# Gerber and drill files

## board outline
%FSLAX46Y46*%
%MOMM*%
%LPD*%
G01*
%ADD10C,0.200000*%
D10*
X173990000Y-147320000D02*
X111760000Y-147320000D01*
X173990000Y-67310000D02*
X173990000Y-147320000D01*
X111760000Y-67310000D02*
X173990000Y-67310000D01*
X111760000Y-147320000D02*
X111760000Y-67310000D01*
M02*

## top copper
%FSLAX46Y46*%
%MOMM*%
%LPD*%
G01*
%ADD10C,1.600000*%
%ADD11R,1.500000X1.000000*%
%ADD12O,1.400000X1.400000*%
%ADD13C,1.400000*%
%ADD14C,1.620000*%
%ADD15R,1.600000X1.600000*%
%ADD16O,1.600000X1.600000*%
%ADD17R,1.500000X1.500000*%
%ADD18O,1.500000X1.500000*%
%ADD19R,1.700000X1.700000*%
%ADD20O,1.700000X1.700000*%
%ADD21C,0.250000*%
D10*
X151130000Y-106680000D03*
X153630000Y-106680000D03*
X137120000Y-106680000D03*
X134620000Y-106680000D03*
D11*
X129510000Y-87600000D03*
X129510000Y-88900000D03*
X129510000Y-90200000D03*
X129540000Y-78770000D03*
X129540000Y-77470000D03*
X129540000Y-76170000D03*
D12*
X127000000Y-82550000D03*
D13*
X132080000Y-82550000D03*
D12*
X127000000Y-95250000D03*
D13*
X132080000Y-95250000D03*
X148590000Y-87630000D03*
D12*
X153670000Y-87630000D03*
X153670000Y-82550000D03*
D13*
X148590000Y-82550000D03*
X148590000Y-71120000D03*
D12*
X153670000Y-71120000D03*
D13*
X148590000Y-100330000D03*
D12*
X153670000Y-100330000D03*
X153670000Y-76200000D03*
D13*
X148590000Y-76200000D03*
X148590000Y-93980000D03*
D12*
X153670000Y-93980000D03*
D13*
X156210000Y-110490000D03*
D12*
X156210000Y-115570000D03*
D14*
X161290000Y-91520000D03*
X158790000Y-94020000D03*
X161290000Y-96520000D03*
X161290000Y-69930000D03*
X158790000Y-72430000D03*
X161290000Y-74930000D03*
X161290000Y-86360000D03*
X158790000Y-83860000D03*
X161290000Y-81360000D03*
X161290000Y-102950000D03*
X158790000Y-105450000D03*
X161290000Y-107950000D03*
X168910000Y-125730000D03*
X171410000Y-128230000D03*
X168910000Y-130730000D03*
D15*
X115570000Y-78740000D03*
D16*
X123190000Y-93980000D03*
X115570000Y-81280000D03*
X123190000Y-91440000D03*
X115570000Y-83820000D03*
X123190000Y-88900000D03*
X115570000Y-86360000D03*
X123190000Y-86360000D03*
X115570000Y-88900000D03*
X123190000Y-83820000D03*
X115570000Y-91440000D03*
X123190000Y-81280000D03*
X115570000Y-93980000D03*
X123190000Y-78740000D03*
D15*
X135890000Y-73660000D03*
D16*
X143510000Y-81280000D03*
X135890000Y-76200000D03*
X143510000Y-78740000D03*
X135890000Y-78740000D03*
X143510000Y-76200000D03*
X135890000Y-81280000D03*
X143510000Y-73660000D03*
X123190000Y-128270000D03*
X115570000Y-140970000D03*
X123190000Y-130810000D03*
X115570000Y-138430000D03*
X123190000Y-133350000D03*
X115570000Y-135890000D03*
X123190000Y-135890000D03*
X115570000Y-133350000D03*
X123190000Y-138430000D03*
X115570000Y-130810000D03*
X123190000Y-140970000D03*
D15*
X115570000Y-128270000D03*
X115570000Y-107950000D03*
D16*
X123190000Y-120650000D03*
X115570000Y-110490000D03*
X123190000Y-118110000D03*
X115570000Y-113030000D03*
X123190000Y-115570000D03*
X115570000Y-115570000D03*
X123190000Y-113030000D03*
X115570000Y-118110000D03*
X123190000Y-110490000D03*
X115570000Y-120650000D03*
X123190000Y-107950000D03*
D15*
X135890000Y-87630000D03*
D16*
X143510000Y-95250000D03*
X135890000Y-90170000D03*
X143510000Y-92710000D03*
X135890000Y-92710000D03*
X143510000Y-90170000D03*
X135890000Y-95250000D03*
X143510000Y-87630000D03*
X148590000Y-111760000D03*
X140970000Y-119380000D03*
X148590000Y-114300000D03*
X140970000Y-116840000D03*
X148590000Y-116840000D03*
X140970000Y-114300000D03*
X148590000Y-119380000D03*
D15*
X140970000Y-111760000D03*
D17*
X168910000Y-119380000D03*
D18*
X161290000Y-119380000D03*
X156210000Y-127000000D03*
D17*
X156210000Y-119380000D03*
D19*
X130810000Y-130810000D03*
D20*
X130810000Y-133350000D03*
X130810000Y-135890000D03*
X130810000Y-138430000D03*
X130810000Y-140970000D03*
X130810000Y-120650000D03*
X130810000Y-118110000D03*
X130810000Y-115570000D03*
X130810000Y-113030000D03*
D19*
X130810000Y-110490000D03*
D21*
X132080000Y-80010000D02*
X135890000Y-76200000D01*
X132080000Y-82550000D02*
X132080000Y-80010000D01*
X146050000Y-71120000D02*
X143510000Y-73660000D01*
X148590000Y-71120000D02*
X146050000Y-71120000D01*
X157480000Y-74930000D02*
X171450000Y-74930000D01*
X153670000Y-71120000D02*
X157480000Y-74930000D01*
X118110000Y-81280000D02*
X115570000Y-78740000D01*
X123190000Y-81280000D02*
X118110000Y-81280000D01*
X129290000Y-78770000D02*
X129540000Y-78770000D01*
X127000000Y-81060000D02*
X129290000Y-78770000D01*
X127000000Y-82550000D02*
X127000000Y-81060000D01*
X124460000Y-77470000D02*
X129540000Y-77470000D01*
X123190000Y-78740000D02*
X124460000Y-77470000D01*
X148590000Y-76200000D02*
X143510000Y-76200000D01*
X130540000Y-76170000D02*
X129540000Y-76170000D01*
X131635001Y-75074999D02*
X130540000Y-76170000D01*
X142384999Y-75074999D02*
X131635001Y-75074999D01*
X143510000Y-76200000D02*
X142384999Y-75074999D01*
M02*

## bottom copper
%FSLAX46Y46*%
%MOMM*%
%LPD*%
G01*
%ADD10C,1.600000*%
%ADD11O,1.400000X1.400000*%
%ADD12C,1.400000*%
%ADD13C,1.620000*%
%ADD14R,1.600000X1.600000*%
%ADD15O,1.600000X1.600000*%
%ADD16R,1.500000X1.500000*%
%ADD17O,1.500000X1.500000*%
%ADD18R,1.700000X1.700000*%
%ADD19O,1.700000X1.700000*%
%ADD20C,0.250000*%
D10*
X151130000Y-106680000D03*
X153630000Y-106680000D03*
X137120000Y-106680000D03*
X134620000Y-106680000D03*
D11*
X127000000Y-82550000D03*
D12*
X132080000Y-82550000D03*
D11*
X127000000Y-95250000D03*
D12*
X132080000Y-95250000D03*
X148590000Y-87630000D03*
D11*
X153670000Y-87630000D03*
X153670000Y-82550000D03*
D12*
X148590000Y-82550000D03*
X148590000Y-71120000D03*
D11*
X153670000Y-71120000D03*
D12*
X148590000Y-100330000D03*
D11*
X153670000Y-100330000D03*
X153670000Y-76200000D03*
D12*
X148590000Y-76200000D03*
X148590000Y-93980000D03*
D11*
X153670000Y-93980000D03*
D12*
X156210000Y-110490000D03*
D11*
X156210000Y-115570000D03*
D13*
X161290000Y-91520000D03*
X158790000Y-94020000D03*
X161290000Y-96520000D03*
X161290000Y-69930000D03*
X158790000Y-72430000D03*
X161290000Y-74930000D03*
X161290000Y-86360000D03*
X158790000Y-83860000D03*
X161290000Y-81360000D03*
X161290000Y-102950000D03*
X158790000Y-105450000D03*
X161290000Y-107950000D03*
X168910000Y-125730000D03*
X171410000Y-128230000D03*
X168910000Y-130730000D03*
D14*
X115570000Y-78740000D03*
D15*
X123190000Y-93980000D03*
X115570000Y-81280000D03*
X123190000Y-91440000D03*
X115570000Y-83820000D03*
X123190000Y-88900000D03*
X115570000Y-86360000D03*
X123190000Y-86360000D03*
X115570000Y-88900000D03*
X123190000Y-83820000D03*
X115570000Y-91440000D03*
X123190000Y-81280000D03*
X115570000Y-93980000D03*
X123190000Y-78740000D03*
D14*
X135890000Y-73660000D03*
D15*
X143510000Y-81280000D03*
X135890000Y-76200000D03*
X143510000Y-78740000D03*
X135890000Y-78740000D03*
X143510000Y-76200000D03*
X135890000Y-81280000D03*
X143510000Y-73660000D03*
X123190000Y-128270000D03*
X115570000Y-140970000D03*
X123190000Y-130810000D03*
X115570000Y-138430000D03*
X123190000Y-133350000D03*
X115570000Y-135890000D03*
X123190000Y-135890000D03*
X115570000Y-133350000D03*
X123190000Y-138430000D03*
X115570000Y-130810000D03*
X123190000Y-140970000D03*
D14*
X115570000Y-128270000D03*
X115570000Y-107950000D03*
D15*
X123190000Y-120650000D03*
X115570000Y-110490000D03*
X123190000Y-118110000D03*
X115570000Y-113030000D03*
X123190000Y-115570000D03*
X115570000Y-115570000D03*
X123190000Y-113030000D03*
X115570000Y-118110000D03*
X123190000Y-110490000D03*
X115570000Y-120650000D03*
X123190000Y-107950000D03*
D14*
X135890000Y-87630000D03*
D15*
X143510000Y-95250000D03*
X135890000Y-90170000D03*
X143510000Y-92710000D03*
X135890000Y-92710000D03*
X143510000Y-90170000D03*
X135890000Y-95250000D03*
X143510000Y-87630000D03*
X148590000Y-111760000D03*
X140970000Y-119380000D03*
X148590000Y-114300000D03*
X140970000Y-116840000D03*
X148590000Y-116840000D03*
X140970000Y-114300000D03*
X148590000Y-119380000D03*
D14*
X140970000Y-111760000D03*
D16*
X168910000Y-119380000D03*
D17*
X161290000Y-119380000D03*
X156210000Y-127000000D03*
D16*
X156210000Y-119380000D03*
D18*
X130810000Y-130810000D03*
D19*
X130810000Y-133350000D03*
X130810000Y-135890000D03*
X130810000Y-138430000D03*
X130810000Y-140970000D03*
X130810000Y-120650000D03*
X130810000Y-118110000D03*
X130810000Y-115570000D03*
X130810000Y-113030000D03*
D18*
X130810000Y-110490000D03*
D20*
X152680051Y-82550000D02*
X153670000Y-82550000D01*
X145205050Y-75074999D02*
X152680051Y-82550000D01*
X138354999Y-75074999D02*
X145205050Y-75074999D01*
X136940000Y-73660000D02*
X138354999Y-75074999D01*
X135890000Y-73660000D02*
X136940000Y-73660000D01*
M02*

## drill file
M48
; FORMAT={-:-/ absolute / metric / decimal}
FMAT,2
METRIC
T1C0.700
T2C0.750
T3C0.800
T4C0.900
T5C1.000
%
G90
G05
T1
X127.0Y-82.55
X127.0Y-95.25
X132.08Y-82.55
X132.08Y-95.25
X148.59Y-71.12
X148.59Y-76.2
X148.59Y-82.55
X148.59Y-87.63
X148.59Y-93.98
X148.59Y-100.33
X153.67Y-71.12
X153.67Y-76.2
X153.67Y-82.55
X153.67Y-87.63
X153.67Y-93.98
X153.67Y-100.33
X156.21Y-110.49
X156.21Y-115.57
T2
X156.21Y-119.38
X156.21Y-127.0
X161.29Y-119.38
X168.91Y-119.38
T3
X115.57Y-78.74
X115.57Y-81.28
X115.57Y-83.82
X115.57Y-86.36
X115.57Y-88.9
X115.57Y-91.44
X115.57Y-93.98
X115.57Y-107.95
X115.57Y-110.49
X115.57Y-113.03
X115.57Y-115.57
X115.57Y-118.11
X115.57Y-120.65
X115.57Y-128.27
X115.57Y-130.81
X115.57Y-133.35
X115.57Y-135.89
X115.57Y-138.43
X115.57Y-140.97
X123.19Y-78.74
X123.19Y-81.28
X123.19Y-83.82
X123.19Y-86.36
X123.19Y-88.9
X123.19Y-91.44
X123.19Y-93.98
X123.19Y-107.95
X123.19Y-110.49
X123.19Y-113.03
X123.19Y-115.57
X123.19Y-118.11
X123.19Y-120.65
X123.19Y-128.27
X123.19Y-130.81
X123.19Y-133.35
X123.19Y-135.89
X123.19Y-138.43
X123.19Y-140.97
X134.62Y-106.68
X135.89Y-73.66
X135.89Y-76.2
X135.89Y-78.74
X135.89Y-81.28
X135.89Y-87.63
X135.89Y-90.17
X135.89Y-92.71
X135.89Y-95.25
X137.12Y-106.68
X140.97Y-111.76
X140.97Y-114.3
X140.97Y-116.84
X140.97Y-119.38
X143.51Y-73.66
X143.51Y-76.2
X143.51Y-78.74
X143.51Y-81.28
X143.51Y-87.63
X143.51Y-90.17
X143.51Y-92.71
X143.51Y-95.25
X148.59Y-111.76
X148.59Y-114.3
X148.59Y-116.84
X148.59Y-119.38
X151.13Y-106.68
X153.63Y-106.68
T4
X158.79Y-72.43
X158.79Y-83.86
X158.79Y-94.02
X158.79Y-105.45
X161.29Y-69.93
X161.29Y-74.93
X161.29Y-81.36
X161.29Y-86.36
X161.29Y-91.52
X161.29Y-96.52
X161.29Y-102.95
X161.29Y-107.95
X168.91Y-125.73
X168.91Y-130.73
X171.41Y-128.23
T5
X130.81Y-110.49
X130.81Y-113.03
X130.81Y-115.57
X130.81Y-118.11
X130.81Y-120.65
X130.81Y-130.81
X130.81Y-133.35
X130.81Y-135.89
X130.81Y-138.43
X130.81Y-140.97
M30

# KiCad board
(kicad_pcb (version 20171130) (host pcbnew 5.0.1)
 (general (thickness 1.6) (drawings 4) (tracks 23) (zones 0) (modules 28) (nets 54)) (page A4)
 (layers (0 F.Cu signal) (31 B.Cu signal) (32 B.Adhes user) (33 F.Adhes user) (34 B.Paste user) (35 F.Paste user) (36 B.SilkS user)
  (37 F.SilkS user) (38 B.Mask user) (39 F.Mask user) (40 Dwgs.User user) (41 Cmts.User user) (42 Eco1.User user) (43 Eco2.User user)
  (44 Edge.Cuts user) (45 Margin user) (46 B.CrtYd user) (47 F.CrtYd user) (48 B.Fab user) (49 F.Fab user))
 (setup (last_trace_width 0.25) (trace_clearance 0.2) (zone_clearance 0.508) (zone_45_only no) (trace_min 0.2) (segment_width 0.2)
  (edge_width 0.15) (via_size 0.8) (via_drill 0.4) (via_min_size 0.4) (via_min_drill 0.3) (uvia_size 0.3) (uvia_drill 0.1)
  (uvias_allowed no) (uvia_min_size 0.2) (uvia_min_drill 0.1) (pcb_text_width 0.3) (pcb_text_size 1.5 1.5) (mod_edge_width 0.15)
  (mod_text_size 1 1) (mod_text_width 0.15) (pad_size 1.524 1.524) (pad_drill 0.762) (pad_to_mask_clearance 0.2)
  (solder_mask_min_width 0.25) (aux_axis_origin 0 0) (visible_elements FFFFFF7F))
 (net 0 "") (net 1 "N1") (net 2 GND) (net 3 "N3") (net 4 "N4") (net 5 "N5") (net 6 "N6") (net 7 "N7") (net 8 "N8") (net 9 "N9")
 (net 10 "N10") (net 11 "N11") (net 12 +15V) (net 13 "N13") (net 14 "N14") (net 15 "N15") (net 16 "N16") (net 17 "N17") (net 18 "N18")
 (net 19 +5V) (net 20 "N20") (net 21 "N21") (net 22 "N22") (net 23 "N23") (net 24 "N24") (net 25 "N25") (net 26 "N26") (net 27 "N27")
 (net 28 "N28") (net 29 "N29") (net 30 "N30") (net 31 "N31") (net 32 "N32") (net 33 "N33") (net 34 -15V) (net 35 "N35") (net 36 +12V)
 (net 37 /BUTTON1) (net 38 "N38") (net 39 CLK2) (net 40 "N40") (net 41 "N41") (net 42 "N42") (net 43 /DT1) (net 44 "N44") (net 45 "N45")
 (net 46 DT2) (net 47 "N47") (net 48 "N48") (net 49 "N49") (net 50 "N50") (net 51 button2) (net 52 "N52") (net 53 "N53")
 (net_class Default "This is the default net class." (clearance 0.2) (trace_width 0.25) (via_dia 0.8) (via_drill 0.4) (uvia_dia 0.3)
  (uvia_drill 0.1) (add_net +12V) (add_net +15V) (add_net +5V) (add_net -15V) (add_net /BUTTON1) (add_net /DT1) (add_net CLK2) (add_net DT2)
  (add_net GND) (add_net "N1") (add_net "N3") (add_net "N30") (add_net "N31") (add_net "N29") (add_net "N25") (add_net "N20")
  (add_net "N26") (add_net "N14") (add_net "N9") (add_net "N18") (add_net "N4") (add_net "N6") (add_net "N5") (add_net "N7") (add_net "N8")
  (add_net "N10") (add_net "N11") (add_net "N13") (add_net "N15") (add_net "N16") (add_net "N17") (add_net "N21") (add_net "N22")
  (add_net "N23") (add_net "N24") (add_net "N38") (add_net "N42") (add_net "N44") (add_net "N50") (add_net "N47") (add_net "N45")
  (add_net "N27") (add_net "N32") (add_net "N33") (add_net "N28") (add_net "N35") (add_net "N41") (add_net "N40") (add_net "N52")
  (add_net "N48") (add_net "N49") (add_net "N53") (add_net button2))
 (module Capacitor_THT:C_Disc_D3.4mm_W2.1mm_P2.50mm (layer F.Cu) (at 151.13 106.68)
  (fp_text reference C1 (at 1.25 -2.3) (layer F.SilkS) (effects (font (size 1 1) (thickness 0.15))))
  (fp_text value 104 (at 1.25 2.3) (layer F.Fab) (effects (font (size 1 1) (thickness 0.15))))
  (pad 1 thru_hole circle (at 0 0) (size 1.6 1.6) (drill 0.8) (layers *.Cu *.Mask) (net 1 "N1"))
  (pad 2 thru_hole circle (at 2.5 0) (size 1.6 1.6) (drill 0.8) (layers *.Cu *.Mask) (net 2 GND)))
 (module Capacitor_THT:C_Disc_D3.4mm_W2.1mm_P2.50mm (layer F.Cu) (at 134.62 106.68)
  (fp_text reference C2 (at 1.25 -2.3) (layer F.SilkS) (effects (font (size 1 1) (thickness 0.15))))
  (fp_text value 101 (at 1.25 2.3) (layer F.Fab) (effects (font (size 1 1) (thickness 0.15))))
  (pad 2 thru_hole circle (at 2.5 0) (size 1.6 1.6) (drill 0.8) (layers *.Cu *.Mask) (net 2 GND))
  (pad 1 thru_hole circle (at 0 0) (size 1.6 1.6) (drill 0.8) (layers *.Cu *.Mask) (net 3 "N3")))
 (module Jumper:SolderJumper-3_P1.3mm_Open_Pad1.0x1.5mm (layer F.Cu) (at 129.51 88.9 90)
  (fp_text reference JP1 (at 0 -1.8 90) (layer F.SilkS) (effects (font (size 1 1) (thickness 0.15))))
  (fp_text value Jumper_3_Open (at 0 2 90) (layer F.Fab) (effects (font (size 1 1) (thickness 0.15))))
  (pad 3 smd rect (at 1.3 0 90) (size 1 1.5) (layers F.Cu F.Mask) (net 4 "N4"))
  (pad 2 smd rect (at 0 0 90) (size 1 1.5) (layers F.Cu F.Mask) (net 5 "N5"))
  (pad 1 smd rect (at -1.3 0 90) (size 1 1.5) (layers F.Cu F.Mask) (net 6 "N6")))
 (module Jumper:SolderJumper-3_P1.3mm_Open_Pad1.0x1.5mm (layer F.Cu) (at 129.54 77.47 90)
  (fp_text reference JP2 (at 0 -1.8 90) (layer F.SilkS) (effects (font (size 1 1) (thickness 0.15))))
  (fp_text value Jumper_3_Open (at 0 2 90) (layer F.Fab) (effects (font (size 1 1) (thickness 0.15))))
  (pad 1 smd rect (at -1.3 0 90) (size 1 1.5) (layers F.Cu F.Mask) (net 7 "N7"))
  (pad 2 smd rect (at 0 0 90) (size 1 1.5) (layers F.Cu F.Mask) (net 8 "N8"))
  (pad 3 smd rect (at 1.3 0 90) (size 1 1.5) (layers F.Cu F.Mask) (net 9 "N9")))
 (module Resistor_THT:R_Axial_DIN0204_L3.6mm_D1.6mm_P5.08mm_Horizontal (layer F.Cu) (at 132.08 82.55 180)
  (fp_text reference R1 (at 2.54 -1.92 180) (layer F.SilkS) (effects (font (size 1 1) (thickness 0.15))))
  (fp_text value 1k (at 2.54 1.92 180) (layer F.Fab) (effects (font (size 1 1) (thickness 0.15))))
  (pad 2 thru_hole oval (at 5.08 0 180) (size 1.4 1.4) (drill 0.7) (layers *.Cu *.Mask) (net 7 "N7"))
  (pad 1 thru_hole circle (at 0 0 180) (size 1.4 1.4) (drill 0.7) (layers *.Cu *.Mask) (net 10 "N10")))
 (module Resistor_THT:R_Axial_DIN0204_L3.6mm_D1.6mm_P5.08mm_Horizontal (layer F.Cu) (at 132.08 95.25 180)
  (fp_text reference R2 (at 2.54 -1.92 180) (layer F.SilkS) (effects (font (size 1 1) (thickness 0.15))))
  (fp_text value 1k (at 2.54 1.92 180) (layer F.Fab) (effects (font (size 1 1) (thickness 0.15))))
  (pad 2 thru_hole oval (at 5.08 0 180) (size 1.4 1.4) (drill 0.7) (layers *.Cu *.Mask) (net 6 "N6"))
  (pad 1 thru_hole circle (at 0 0 180) (size 1.4 1.4) (drill 0.7) (layers *.Cu *.Mask) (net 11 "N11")))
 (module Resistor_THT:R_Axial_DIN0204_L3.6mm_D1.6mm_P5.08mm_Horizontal (layer F.Cu) (at 148.59 87.63)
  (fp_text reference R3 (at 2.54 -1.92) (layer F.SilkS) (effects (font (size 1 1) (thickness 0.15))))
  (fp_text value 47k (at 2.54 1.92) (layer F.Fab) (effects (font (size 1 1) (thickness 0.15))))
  (pad 1 thru_hole circle (at 0 0) (size 1.4 1.4) (drill 0.7) (layers *.Cu *.Mask) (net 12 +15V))
  (pad 2 thru_hole oval (at 5.08 0) (size 1.4 1.4) (drill 0.7) (layers *.Cu *.Mask) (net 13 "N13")))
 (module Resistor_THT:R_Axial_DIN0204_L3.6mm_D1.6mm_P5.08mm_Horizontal (layer F.Cu) (at 148.59 82.55)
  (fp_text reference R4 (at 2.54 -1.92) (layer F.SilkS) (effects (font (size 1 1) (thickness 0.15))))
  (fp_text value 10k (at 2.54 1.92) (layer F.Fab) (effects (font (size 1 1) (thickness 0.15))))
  (pad 2 thru_hole oval (at 5.08 0) (size 1.4 1.4) (drill 0.7) (layers *.Cu *.Mask) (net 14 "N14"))
  (pad 1 thru_hole circle (at 0 0) (size 1.4 1.4) (drill 0.7) (layers *.Cu *.Mask) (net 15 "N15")))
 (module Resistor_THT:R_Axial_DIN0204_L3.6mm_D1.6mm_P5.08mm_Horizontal (layer F.Cu) (at 148.59 71.12)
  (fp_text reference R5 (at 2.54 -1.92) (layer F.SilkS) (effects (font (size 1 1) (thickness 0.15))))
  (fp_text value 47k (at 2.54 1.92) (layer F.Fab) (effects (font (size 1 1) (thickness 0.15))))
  (pad 1 thru_hole circle (at 0 0) (size 1.4 1.4) (drill 0.7) (layers *.Cu *.Mask) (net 12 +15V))
  (pad 2 thru_hole oval (at 5.08 0) (size 1.4 1.4) (drill 0.7) (layers *.Cu *.Mask) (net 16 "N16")))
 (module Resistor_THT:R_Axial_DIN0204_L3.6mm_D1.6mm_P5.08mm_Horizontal (layer F.Cu) (at 148.59 100.33)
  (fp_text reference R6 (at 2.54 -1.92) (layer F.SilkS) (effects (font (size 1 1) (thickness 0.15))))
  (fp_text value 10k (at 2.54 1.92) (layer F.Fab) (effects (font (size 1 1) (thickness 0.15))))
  (pad 1 thru_hole circle (at 0 0) (size 1.4 1.4) (drill 0.7) (layers *.Cu *.Mask) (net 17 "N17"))
  (pad 2 thru_hole oval (at 5.08 0) (size 1.4 1.4) (drill 0.7) (layers *.Cu *.Mask) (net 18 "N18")))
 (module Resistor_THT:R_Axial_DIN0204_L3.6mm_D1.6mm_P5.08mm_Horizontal (layer F.Cu) (at 148.59 76.2)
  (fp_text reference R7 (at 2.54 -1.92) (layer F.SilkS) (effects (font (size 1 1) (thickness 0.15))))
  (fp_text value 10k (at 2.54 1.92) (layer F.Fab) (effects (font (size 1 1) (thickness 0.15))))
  (pad 2 thru_hole oval (at 5.08 0) (size 1.4 1.4) (drill 0.7) (layers *.Cu *.Mask) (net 15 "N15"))
  (pad 1 thru_hole circle (at 0 0) (size 1.4 1.4) (drill 0.7) (layers *.Cu *.Mask) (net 9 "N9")))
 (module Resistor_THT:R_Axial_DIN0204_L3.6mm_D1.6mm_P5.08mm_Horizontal (layer F.Cu) (at 148.59 93.98)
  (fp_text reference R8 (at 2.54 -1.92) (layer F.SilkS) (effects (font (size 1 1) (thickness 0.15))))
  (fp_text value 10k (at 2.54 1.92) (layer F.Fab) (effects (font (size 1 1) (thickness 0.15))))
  (pad 1 thru_hole circle (at 0 0) (size 1.4 1.4) (drill 0.7) (layers *.Cu *.Mask) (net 4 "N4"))
  (pad 2 thru_hole oval (at 5.08 0) (size 1.4 1.4) (drill 0.7) (layers *.Cu *.Mask) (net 17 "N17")))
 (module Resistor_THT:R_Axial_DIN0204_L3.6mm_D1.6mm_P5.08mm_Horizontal (layer F.Cu) (at 156.21 110.49 270)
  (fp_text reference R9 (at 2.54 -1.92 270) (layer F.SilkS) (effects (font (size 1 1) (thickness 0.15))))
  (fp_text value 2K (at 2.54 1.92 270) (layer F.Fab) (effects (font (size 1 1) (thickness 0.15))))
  (pad 1 thru_hole circle (at 0 0 270) (size 1.4 1.4) (drill 0.7) (layers *.Cu *.Mask) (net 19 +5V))
  (pad 2 thru_hole oval (at 5.08 0 270) (size 1.4 1.4) (drill 0.7) (layers *.Cu *.Mask) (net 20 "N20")))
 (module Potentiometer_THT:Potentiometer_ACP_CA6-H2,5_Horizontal (layer F.Cu) (at 161.29 96.52 180)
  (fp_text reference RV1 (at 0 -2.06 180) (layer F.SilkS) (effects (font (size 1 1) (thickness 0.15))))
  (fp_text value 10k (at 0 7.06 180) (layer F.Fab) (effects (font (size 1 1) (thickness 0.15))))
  (pad 3 thru_hole circle (at 0 5 180) (size 1.62 1.62) (drill 0.9) (layers *.Cu *.Mask) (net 2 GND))
  (pad 2 thru_hole circle (at 2.5 2.5 180) (size 1.62 1.62) (drill 0.9) (layers *.Cu *.Mask) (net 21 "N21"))
  (pad 1 thru_hole circle (at 0 0 180) (size 1.62 1.62) (drill 0.9) (layers *.Cu *.Mask) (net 13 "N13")))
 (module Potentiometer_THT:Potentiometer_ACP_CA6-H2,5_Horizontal (layer F.Cu) (at 161.29 74.93 180)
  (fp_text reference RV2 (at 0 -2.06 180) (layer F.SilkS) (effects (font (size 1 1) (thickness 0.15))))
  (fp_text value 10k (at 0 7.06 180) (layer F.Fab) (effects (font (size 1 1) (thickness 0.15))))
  (pad 3 thru_hole circle (at 0 5 180) (size 1.62 1.62) (drill 0.9) (layers *.Cu *.Mask) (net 2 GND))
  (pad 2 thru_hole circle (at 2.5 2.5 180) (size 1.62 1.62) (drill 0.9) (layers *.Cu *.Mask) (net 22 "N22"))
  (pad 1 thru_hole circle (at 0 0 180) (size 1.62 1.62) (drill 0.9) (layers *.Cu *.Mask) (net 16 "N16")))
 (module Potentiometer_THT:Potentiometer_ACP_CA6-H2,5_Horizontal (layer F.Cu) (at 161.29 86.36 180)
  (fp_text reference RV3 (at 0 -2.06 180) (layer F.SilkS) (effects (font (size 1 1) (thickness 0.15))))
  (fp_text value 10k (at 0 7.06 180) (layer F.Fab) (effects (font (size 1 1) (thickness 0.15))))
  (pad 1 thru_hole circle (at 0 0 180) (size 1.62 1.62) (drill 0.9) (layers *.Cu *.Mask) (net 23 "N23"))
  (pad 2 thru_hole circle (at 2.5 2.5 180) (size 1.62 1.62) (drill 0.9) (layers *.Cu *.Mask) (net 14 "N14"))
  (pad 3 thru_hole circle (at 0 5 180) (size 1.62 1.62) (drill 0.9) (layers *.Cu *.Mask) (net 10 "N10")))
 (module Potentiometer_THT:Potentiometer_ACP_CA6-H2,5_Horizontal (layer F.Cu) (at 161.29 107.95 180)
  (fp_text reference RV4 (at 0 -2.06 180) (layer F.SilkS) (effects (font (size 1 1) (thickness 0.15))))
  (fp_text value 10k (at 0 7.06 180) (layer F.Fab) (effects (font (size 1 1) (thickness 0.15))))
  (pad 3 thru_hole circle (at 0 5 180) (size 1.62 1.62) (drill 0.9) (layers *.Cu *.Mask) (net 11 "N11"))
  (pad 2 thru_hole circle (at 2.5 2.5 180) (size 1.62 1.62) (drill 0.9) (layers *.Cu *.Mask) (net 18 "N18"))
  (pad 1 thru_hole circle (at 0 0 180) (size 1.62 1.62) (drill 0.9) (layers *.Cu *.Mask) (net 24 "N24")))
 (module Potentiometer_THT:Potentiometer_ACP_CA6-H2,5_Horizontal (layer F.Cu) (at 168.91 125.73)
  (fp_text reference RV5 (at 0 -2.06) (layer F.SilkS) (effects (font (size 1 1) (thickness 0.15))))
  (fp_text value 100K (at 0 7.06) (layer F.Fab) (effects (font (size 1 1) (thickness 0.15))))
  (pad 1 thru_hole circle (at 0 0) (size 1.62 1.62) (drill 0.9) (layers *.Cu *.Mask) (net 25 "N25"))
  (pad 2 thru_hole circle (at 2.5 2.5) (size 1.62 1.62) (drill 0.9) (layers *.Cu *.Mask) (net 3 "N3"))
  (pad 3 thru_hole circle (at 0 5) (size 1.62 1.62) (drill 0.9) (layers *.Cu *.Mask) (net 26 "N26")))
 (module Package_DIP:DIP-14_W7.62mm (layer F.Cu) (at 115.57 78.74)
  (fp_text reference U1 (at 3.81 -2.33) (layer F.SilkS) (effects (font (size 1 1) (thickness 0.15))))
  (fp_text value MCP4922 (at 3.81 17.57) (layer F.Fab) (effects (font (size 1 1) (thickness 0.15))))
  (pad 1 thru_hole rect (at 0 0) (size 1.6 1.6) (drill 0.8) (layers *.Cu *.Mask) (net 19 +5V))
  (pad 8 thru_hole oval (at 7.62 15.24) (size 1.6 1.6) (drill 0.8) (layers *.Cu *.Mask) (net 2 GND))
  (pad 2 thru_hole oval (at 0 2.54) (size 1.6 1.6) (drill 0.8) (layers *.Cu *.Mask) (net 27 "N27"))
  (pad 9 thru_hole oval (at 7.62 12.7) (size 1.6 1.6) (drill 0.8) (layers *.Cu *.Mask) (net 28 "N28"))
  (pad 3 thru_hole oval (at 0 5.08) (size 1.6 1.6) (drill 0.8) (layers *.Cu *.Mask) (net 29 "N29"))
  (pad 10 thru_hole oval (at 7.62 10.16) (size 1.6 1.6) (drill 0.8) (layers *.Cu *.Mask) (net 5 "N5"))
  (pad 4 thru_hole oval (at 0 7.62) (size 1.6 1.6) (drill 0.8) (layers *.Cu *.Mask) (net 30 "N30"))
  (pad 11 thru_hole oval (at 7.62 7.62) (size 1.6 1.6) (drill 0.8) (layers *.Cu *.Mask) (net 19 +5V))
  (pad 5 thru_hole oval (at 0 10.16) (size 1.6 1.6) (drill 0.8) (layers *.Cu *.Mask) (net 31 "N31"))
  (pad 12 thru_hole oval (at 7.62 5.08) (size 1.6 1.6) (drill 0.8) (layers *.Cu *.Mask) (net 2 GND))
  (pad 6 thru_hole oval (at 0 12.7) (size 1.6 1.6) (drill 0.8) (layers *.Cu *.Mask) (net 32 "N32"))
  (pad 13 thru_hole oval (at 7.62 2.54) (size 1.6 1.6) (drill 0.8) (layers *.Cu *.Mask) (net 19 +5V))
  (pad 7 thru_hole oval (at 0 15.24) (size 1.6 1.6) (drill 0.8) (layers *.Cu *.Mask) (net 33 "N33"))
  (pad 14 thru_hole oval (at 7.62 0) (size 1.6 1.6) (drill 0.8) (layers *.Cu *.Mask) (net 8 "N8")))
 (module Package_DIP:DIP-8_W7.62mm (layer F.Cu) (at 135.89 73.66)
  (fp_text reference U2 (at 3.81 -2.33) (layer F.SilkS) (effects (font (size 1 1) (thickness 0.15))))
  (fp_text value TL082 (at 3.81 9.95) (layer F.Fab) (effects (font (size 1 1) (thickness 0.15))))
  (pad 1 thru_hole rect (at 0 0) (size 1.6 1.6) (drill 0.8) (layers *.Cu *.Mask) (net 14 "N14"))
  (pad 5 thru_hole oval (at 7.62 7.62) (size 1.6 1.6) (drill 0.8) (layers *.Cu *.Mask) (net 2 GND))
  (pad 2 thru_hole oval (at 0 2.54) (size 1.6 1.6) (drill 0.8) (layers *.Cu *.Mask) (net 10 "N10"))
  (pad 6 thru_hole oval (at 7.62 5.08) (size 1.6 1.6) (drill 0.8) (layers *.Cu *.Mask) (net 15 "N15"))
  (pad 3 thru_hole oval (at 0 5.08) (size 1.6 1.6) (drill 0.8) (layers *.Cu *.Mask) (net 21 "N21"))
  (pad 7 thru_hole oval (at 7.62 2.54) (size 1.6 1.6) (drill 0.8) (layers *.Cu *.Mask) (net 9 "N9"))
  (pad 4 thru_hole oval (at 0 7.62) (size 1.6 1.6) (drill 0.8) (layers *.Cu *.Mask) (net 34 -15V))
  (pad 8 thru_hole oval (at 7.62 0) (size 1.6 1.6) (drill 0.8) (layers *.Cu *.Mask) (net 12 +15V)))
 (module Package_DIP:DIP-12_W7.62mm (layer F.Cu) (at 115.57 128.27)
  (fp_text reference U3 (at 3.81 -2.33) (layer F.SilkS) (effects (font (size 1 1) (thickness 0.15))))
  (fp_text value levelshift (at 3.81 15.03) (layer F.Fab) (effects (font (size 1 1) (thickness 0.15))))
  (pad 12 thru_hole oval (at 7.62 0) (size 1.6 1.6) (drill 0.8) (layers *.Cu *.Mask) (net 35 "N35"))
  (pad 6 thru_hole oval (at 0 12.7) (size 1.6 1.6) (drill 0.8) (layers *.Cu *.Mask) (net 2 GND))
  (pad 11 thru_hole oval (at 7.62 2.54) (size 1.6 1.6) (drill 0.8) (layers *.Cu *.Mask) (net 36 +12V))
  (pad 5 thru_hole oval (at 0 10.16) (size 1.6 1.6) (drill 0.8) (layers *.Cu *.Mask) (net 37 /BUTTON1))
  (pad 10 thru_hole oval (at 7.62 5.08) (size 1.6 1.6) (drill 0.8) (layers *.Cu *.Mask) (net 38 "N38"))
  (pad 4 thru_hole oval (at 0 7.62) (size 1.6 1.6) (drill 0.8) (layers *.Cu *.Mask) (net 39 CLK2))
  (pad 9 thru_hole oval (at 7.62 7.62) (size 1.6 1.6) (drill 0.8) (layers *.Cu *.Mask) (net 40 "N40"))
  (pad 3 thru_hole oval (at 0 5.08) (size 1.6 1.6) (drill 0.8) (layers *.Cu *.Mask) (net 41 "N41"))
  (pad 8 thru_hole oval (at 7.62 10.16) (size 1.6 1.6) (drill 0.8) (layers *.Cu *.Mask) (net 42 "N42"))
  (pad 2 thru_hole oval (at 0 2.54) (size 1.6 1.6) (drill 0.8) (layers *.Cu *.Mask) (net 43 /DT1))
  (pad 7 thru_hole oval (at 7.62 12.7) (size 1.6 1.6) (drill 0.8) (layers *.Cu *.Mask) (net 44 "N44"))
  (pad 1 thru_hole rect (at 0 0) (size 1.6 1.6) (drill 0.8) (layers *.Cu *.Mask) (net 19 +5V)))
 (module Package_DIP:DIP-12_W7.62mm (layer F.Cu) (at 115.57 107.95)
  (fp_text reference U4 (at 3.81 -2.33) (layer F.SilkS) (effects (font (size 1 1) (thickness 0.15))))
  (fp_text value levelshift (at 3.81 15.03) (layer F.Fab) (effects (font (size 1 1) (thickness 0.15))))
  (pad 1 thru_hole rect (at 0 0) (size 1.6 1.6) (drill 0.8) (layers *.Cu *.Mask) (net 19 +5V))
  (pad 7 thru_hole oval (at 7.62 12.7) (size 1.6 1.6) (drill 0.8) (layers *.Cu *.Mask) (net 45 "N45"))
  (pad 2 thru_hole oval (at 0 2.54) (size 1.6 1.6) (drill 0.8) (layers *.Cu *.Mask) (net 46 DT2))
  (pad 8 thru_hole oval (at 7.62 10.16) (size 1.6 1.6) (drill 0.8) (layers *.Cu *.Mask) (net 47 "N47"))
  (pad 3 thru_hole oval (at 0 5.08) (size 1.6 1.6) (drill 0.8) (layers *.Cu *.Mask) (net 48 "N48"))
  (pad 9 thru_hole oval (at 7.62 7.62) (size 1.6 1.6) (drill 0.8) (layers *.Cu *.Mask) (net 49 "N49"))
  (pad 4 thru_hole oval (at 0 7.62) (size 1.6 1.6) (drill 0.8) (layers *.Cu *.Mask) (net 39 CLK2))
  (pad 10 thru_hole oval (at 7.62 5.08) (size 1.6 1.6) (drill 0.8) (layers *.Cu *.Mask) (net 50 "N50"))
  (pad 5 thru_hole oval (at 0 10.16) (size 1.6 1.6) (drill 0.8) (layers *.Cu *.Mask) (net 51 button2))
  (pad 11 thru_hole oval (at 7.62 2.54) (size 1.6 1.6) (drill 0.8) (layers *.Cu *.Mask) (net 36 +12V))
  (pad 6 thru_hole oval (at 0 12.7) (size 1.6 1.6) (drill 0.8) (layers *.Cu *.Mask) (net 2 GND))
  (pad 12 thru_hole oval (at 7.62 0) (size 1.6 1.6) (drill 0.8) (layers *.Cu *.Mask) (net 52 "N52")))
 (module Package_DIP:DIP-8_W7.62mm (layer F.Cu) (at 135.89 87.63)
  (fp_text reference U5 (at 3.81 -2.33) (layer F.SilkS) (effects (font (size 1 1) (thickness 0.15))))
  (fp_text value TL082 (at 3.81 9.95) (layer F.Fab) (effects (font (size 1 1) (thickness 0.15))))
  (pad 1 thru_hole rect (at 0 0) (size 1.6 1.6) (drill 0.8) (layers *.Cu *.Mask) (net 18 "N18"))
  (pad 5 thru_hole oval (at 7.62 7.62) (size 1.6 1.6) (drill 0.8) (layers *.Cu *.Mask) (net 2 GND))
  (pad 2 thru_hole oval (at 0 2.54) (size 1.6 1.6) (drill 0.8) (layers *.Cu *.Mask) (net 11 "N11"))
  (pad 6 thru_hole oval (at 7.62 5.08) (size 1.6 1.6) (drill 0.8) (layers *.Cu *.Mask) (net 17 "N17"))
  (pad 3 thru_hole oval (at 0 5.08) (size 1.6 1.6) (drill 0.8) (layers *.Cu *.Mask) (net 22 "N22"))
  (pad 7 thru_hole oval (at 7.62 2.54) (size 1.6 1.6) (drill 0.8) (layers *.Cu *.Mask) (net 4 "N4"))
  (pad 4 thru_hole oval (at 0 7.62) (size 1.6 1.6) (drill 0.8) (layers *.Cu *.Mask) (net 34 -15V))
  (pad 8 thru_hole oval (at 7.62 0) (size 1.6 1.6) (drill 0.8) (layers *.Cu *.Mask) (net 12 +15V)))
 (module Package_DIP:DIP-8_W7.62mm (layer F.Cu) (at 140.97 111.76)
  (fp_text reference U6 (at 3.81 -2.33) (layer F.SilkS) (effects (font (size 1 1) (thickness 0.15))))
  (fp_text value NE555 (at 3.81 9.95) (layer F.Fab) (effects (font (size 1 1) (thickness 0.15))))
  (pad 8 thru_hole oval (at 7.62 0) (size 1.6 1.6) (drill 0.8) (layers *.Cu *.Mask) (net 19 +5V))
  (pad 4 thru_hole oval (at 0 7.62) (size 1.6 1.6) (drill 0.8) (layers *.Cu *.Mask) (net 19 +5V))
  (pad 7 thru_hole oval (at 7.62 2.54) (size 1.6 1.6) (drill 0.8) (layers *.Cu *.Mask) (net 20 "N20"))
  (pad 3 thru_hole oval (at 0 5.08) (size 1.6 1.6) (drill 0.8) (layers *.Cu *.Mask) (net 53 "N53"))
  (pad 6 thru_hole oval (at 7.62 5.08) (size 1.6 1.6) (drill 0.8) (layers *.Cu *.Mask) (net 3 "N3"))
  (pad 2 thru_hole oval (at 0 2.54) (size 1.6 1.6) (drill 0.8) (layers *.Cu *.Mask) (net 3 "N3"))
  (pad 5 thru_hole oval (at 7.62 7.62) (size 1.6 1.6) (drill 0.8) (layers *.Cu *.Mask) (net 1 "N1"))
  (pad 1 thru_hole rect (at 0 0) (size 1.6 1.6) (drill 0.8) (layers *.Cu *.Mask) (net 2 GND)))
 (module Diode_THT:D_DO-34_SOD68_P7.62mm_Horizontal (layer F.Cu) (at 168.91 119.38 180)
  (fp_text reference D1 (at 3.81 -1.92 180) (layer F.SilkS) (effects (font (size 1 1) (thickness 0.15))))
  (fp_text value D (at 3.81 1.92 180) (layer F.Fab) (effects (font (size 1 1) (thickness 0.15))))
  (pad 1 thru_hole rect (at 0 0 180) (size 1.5 1.5) (drill 0.75) (layers *.Cu *.Mask) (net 25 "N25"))
  (pad 2 thru_hole oval (at 7.62 0 180) (size 1.5 1.5) (drill 0.75) (layers *.Cu *.Mask) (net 20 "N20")))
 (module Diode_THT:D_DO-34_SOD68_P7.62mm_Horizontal (layer F.Cu) (at 156.21 119.38 270)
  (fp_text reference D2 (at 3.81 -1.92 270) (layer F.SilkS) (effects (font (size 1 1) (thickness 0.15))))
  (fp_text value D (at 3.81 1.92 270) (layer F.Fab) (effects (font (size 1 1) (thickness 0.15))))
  (pad 2 thru_hole oval (at 7.62 0 270) (size 1.5 1.5) (drill 0.75) (layers *.Cu *.Mask) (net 26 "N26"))
  (pad 1 thru_hole rect (at 0 0 270) (size 1.5 1.5) (drill 0.75) (layers *.Cu *.Mask) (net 20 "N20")))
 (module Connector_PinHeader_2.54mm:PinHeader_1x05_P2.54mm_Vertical (layer F.Cu) (at 130.81 130.81)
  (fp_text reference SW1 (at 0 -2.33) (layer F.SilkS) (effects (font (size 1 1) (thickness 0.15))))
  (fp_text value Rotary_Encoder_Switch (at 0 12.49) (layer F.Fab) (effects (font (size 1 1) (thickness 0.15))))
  (pad 1 thru_hole rect (at 0 0) (size 1.7 1.7) (drill 1) (layers *.Cu *.Mask) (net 38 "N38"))
  (pad 2 thru_hole oval (at 0 2.54) (size 1.7 1.7) (drill 1) (layers *.Cu *.Mask) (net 36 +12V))
  (pad 3 thru_hole oval (at 0 5.08) (size 1.7 1.7) (drill 1) (layers *.Cu *.Mask) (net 42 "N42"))
  (pad 4 thru_hole oval (at 0 7.62) (size 1.7 1.7) (drill 1) (layers *.Cu *.Mask) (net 2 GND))
  (pad 5 thru_hole oval (at 0 10.16) (size 1.7 1.7) (drill 1) (layers *.Cu *.Mask) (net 44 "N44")))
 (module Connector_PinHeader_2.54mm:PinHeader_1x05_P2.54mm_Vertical (layer F.Cu) (at 130.81 110.49)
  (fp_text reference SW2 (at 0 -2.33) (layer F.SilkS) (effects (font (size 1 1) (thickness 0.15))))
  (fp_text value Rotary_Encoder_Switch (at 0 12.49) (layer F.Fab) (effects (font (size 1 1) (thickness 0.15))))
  (pad 5 thru_hole oval (at 0 10.16) (size 1.7 1.7) (drill 1) (layers *.Cu *.Mask) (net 45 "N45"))
  (pad 4 thru_hole oval (at 0 7.62) (size 1.7 1.7) (drill 1) (layers *.Cu *.Mask) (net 2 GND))
  (pad 3 thru_hole oval (at 0 5.08) (size 1.7 1.7) (drill 1) (layers *.Cu *.Mask) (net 47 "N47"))
  (pad 2 thru_hole oval (at 0 2.54) (size 1.7 1.7) (drill 1) (layers *.Cu *.Mask) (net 36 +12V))
  (pad 1 thru_hole rect (at 0 0) (size 1.7 1.7) (drill 1) (layers *.Cu *.Mask) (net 50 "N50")))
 (gr_line (start 173.99 147.32) (end 111.76 147.32) (layer Edge.Cuts) (width 0.2))
 (gr_line (start 173.99 67.31) (end 173.99 147.32) (layer Edge.Cuts) (width 0.2))
 (gr_line (start 111.76 67.31) (end 173.99 67.31) (layer Edge.Cuts) (width 0.2))
 (gr_line (start 111.76 147.32) (end 111.76 67.31) (layer Edge.Cuts) (width 0.2))
 (segment (start 132.08 80.01) (end 135.89 76.2) (width 0.25) (layer F.Cu) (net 10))
 (segment (start 132.08 82.55) (end 132.08 80.01) (width 0.25) (layer F.Cu) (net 10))
 (segment (start 146.05 71.12) (end 143.51 73.66) (width 0.25) (layer F.Cu) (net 12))
 (segment (start 148.59 71.12) (end 146.05 71.12) (width 0.25) (layer F.Cu) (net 12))
 (segment (start 157.48 74.93) (end 171.45 74.93) (width 0.25) (layer F.Cu) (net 16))
 (segment (start 153.67 71.12) (end 157.48 74.93) (width 0.25) (layer F.Cu) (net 16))
 (segment (start 118.11 81.28) (end 115.57 78.74) (width 0.25) (layer F.Cu) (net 19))
 (segment (start 123.19 81.28) (end 118.11 81.28) (width 0.25) (layer F.Cu) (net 19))
 (segment (start 129.29 78.77) (end 129.54 78.77) (width 0.25) (layer F.Cu) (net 7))
 (segment (start 127 81.06) (end 129.29 78.77) (width 0.25) (layer F.Cu) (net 7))
 (segment (start 127 82.55) (end 127 81.06) (width 0.25) (layer F.Cu) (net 7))
 (segment (start 124.46 77.47) (end 129.54 77.47) (width 0.25) (layer F.Cu) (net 8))
 (segment (start 123.19 78.74) (end 124.46 77.47) (width 0.25) (layer F.Cu) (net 8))
 (segment (start 148.59 76.2) (end 143.51 76.2) (width 0.25) (layer F.Cu) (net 9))
 (segment (start 130.54 76.17) (end 129.54 76.17) (width 0.25) (layer F.Cu) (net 9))
 (segment (start 131.635001 75.074999) (end 130.54 76.17) (width 0.25) (layer F.Cu) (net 9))
 (segment (start 142.384999 75.074999) (end 131.635001 75.074999) (width 0.25) (layer F.Cu) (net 9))
 (segment (start 143.51 76.2) (end 142.384999 75.074999) (width 0.25) (layer F.Cu) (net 9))
 (segment (start 152.680051 82.55) (end 153.67 82.55) (width 0.25) (layer B.Cu) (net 14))
 (segment (start 145.20505 75.074999) (end 152.680051 82.55) (width 0.25) (layer B.Cu) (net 14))
 (segment (start 138.354999 75.074999) (end 145.20505 75.074999) (width 0.25) (layer B.Cu) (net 14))
 (segment (start 136.94 73.66) (end 138.354999 75.074999) (width 0.25) (layer B.Cu) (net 14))
 (segment (start 135.89 73.66) (end 136.94 73.66) (width 0.25) (layer B.Cu) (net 14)))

